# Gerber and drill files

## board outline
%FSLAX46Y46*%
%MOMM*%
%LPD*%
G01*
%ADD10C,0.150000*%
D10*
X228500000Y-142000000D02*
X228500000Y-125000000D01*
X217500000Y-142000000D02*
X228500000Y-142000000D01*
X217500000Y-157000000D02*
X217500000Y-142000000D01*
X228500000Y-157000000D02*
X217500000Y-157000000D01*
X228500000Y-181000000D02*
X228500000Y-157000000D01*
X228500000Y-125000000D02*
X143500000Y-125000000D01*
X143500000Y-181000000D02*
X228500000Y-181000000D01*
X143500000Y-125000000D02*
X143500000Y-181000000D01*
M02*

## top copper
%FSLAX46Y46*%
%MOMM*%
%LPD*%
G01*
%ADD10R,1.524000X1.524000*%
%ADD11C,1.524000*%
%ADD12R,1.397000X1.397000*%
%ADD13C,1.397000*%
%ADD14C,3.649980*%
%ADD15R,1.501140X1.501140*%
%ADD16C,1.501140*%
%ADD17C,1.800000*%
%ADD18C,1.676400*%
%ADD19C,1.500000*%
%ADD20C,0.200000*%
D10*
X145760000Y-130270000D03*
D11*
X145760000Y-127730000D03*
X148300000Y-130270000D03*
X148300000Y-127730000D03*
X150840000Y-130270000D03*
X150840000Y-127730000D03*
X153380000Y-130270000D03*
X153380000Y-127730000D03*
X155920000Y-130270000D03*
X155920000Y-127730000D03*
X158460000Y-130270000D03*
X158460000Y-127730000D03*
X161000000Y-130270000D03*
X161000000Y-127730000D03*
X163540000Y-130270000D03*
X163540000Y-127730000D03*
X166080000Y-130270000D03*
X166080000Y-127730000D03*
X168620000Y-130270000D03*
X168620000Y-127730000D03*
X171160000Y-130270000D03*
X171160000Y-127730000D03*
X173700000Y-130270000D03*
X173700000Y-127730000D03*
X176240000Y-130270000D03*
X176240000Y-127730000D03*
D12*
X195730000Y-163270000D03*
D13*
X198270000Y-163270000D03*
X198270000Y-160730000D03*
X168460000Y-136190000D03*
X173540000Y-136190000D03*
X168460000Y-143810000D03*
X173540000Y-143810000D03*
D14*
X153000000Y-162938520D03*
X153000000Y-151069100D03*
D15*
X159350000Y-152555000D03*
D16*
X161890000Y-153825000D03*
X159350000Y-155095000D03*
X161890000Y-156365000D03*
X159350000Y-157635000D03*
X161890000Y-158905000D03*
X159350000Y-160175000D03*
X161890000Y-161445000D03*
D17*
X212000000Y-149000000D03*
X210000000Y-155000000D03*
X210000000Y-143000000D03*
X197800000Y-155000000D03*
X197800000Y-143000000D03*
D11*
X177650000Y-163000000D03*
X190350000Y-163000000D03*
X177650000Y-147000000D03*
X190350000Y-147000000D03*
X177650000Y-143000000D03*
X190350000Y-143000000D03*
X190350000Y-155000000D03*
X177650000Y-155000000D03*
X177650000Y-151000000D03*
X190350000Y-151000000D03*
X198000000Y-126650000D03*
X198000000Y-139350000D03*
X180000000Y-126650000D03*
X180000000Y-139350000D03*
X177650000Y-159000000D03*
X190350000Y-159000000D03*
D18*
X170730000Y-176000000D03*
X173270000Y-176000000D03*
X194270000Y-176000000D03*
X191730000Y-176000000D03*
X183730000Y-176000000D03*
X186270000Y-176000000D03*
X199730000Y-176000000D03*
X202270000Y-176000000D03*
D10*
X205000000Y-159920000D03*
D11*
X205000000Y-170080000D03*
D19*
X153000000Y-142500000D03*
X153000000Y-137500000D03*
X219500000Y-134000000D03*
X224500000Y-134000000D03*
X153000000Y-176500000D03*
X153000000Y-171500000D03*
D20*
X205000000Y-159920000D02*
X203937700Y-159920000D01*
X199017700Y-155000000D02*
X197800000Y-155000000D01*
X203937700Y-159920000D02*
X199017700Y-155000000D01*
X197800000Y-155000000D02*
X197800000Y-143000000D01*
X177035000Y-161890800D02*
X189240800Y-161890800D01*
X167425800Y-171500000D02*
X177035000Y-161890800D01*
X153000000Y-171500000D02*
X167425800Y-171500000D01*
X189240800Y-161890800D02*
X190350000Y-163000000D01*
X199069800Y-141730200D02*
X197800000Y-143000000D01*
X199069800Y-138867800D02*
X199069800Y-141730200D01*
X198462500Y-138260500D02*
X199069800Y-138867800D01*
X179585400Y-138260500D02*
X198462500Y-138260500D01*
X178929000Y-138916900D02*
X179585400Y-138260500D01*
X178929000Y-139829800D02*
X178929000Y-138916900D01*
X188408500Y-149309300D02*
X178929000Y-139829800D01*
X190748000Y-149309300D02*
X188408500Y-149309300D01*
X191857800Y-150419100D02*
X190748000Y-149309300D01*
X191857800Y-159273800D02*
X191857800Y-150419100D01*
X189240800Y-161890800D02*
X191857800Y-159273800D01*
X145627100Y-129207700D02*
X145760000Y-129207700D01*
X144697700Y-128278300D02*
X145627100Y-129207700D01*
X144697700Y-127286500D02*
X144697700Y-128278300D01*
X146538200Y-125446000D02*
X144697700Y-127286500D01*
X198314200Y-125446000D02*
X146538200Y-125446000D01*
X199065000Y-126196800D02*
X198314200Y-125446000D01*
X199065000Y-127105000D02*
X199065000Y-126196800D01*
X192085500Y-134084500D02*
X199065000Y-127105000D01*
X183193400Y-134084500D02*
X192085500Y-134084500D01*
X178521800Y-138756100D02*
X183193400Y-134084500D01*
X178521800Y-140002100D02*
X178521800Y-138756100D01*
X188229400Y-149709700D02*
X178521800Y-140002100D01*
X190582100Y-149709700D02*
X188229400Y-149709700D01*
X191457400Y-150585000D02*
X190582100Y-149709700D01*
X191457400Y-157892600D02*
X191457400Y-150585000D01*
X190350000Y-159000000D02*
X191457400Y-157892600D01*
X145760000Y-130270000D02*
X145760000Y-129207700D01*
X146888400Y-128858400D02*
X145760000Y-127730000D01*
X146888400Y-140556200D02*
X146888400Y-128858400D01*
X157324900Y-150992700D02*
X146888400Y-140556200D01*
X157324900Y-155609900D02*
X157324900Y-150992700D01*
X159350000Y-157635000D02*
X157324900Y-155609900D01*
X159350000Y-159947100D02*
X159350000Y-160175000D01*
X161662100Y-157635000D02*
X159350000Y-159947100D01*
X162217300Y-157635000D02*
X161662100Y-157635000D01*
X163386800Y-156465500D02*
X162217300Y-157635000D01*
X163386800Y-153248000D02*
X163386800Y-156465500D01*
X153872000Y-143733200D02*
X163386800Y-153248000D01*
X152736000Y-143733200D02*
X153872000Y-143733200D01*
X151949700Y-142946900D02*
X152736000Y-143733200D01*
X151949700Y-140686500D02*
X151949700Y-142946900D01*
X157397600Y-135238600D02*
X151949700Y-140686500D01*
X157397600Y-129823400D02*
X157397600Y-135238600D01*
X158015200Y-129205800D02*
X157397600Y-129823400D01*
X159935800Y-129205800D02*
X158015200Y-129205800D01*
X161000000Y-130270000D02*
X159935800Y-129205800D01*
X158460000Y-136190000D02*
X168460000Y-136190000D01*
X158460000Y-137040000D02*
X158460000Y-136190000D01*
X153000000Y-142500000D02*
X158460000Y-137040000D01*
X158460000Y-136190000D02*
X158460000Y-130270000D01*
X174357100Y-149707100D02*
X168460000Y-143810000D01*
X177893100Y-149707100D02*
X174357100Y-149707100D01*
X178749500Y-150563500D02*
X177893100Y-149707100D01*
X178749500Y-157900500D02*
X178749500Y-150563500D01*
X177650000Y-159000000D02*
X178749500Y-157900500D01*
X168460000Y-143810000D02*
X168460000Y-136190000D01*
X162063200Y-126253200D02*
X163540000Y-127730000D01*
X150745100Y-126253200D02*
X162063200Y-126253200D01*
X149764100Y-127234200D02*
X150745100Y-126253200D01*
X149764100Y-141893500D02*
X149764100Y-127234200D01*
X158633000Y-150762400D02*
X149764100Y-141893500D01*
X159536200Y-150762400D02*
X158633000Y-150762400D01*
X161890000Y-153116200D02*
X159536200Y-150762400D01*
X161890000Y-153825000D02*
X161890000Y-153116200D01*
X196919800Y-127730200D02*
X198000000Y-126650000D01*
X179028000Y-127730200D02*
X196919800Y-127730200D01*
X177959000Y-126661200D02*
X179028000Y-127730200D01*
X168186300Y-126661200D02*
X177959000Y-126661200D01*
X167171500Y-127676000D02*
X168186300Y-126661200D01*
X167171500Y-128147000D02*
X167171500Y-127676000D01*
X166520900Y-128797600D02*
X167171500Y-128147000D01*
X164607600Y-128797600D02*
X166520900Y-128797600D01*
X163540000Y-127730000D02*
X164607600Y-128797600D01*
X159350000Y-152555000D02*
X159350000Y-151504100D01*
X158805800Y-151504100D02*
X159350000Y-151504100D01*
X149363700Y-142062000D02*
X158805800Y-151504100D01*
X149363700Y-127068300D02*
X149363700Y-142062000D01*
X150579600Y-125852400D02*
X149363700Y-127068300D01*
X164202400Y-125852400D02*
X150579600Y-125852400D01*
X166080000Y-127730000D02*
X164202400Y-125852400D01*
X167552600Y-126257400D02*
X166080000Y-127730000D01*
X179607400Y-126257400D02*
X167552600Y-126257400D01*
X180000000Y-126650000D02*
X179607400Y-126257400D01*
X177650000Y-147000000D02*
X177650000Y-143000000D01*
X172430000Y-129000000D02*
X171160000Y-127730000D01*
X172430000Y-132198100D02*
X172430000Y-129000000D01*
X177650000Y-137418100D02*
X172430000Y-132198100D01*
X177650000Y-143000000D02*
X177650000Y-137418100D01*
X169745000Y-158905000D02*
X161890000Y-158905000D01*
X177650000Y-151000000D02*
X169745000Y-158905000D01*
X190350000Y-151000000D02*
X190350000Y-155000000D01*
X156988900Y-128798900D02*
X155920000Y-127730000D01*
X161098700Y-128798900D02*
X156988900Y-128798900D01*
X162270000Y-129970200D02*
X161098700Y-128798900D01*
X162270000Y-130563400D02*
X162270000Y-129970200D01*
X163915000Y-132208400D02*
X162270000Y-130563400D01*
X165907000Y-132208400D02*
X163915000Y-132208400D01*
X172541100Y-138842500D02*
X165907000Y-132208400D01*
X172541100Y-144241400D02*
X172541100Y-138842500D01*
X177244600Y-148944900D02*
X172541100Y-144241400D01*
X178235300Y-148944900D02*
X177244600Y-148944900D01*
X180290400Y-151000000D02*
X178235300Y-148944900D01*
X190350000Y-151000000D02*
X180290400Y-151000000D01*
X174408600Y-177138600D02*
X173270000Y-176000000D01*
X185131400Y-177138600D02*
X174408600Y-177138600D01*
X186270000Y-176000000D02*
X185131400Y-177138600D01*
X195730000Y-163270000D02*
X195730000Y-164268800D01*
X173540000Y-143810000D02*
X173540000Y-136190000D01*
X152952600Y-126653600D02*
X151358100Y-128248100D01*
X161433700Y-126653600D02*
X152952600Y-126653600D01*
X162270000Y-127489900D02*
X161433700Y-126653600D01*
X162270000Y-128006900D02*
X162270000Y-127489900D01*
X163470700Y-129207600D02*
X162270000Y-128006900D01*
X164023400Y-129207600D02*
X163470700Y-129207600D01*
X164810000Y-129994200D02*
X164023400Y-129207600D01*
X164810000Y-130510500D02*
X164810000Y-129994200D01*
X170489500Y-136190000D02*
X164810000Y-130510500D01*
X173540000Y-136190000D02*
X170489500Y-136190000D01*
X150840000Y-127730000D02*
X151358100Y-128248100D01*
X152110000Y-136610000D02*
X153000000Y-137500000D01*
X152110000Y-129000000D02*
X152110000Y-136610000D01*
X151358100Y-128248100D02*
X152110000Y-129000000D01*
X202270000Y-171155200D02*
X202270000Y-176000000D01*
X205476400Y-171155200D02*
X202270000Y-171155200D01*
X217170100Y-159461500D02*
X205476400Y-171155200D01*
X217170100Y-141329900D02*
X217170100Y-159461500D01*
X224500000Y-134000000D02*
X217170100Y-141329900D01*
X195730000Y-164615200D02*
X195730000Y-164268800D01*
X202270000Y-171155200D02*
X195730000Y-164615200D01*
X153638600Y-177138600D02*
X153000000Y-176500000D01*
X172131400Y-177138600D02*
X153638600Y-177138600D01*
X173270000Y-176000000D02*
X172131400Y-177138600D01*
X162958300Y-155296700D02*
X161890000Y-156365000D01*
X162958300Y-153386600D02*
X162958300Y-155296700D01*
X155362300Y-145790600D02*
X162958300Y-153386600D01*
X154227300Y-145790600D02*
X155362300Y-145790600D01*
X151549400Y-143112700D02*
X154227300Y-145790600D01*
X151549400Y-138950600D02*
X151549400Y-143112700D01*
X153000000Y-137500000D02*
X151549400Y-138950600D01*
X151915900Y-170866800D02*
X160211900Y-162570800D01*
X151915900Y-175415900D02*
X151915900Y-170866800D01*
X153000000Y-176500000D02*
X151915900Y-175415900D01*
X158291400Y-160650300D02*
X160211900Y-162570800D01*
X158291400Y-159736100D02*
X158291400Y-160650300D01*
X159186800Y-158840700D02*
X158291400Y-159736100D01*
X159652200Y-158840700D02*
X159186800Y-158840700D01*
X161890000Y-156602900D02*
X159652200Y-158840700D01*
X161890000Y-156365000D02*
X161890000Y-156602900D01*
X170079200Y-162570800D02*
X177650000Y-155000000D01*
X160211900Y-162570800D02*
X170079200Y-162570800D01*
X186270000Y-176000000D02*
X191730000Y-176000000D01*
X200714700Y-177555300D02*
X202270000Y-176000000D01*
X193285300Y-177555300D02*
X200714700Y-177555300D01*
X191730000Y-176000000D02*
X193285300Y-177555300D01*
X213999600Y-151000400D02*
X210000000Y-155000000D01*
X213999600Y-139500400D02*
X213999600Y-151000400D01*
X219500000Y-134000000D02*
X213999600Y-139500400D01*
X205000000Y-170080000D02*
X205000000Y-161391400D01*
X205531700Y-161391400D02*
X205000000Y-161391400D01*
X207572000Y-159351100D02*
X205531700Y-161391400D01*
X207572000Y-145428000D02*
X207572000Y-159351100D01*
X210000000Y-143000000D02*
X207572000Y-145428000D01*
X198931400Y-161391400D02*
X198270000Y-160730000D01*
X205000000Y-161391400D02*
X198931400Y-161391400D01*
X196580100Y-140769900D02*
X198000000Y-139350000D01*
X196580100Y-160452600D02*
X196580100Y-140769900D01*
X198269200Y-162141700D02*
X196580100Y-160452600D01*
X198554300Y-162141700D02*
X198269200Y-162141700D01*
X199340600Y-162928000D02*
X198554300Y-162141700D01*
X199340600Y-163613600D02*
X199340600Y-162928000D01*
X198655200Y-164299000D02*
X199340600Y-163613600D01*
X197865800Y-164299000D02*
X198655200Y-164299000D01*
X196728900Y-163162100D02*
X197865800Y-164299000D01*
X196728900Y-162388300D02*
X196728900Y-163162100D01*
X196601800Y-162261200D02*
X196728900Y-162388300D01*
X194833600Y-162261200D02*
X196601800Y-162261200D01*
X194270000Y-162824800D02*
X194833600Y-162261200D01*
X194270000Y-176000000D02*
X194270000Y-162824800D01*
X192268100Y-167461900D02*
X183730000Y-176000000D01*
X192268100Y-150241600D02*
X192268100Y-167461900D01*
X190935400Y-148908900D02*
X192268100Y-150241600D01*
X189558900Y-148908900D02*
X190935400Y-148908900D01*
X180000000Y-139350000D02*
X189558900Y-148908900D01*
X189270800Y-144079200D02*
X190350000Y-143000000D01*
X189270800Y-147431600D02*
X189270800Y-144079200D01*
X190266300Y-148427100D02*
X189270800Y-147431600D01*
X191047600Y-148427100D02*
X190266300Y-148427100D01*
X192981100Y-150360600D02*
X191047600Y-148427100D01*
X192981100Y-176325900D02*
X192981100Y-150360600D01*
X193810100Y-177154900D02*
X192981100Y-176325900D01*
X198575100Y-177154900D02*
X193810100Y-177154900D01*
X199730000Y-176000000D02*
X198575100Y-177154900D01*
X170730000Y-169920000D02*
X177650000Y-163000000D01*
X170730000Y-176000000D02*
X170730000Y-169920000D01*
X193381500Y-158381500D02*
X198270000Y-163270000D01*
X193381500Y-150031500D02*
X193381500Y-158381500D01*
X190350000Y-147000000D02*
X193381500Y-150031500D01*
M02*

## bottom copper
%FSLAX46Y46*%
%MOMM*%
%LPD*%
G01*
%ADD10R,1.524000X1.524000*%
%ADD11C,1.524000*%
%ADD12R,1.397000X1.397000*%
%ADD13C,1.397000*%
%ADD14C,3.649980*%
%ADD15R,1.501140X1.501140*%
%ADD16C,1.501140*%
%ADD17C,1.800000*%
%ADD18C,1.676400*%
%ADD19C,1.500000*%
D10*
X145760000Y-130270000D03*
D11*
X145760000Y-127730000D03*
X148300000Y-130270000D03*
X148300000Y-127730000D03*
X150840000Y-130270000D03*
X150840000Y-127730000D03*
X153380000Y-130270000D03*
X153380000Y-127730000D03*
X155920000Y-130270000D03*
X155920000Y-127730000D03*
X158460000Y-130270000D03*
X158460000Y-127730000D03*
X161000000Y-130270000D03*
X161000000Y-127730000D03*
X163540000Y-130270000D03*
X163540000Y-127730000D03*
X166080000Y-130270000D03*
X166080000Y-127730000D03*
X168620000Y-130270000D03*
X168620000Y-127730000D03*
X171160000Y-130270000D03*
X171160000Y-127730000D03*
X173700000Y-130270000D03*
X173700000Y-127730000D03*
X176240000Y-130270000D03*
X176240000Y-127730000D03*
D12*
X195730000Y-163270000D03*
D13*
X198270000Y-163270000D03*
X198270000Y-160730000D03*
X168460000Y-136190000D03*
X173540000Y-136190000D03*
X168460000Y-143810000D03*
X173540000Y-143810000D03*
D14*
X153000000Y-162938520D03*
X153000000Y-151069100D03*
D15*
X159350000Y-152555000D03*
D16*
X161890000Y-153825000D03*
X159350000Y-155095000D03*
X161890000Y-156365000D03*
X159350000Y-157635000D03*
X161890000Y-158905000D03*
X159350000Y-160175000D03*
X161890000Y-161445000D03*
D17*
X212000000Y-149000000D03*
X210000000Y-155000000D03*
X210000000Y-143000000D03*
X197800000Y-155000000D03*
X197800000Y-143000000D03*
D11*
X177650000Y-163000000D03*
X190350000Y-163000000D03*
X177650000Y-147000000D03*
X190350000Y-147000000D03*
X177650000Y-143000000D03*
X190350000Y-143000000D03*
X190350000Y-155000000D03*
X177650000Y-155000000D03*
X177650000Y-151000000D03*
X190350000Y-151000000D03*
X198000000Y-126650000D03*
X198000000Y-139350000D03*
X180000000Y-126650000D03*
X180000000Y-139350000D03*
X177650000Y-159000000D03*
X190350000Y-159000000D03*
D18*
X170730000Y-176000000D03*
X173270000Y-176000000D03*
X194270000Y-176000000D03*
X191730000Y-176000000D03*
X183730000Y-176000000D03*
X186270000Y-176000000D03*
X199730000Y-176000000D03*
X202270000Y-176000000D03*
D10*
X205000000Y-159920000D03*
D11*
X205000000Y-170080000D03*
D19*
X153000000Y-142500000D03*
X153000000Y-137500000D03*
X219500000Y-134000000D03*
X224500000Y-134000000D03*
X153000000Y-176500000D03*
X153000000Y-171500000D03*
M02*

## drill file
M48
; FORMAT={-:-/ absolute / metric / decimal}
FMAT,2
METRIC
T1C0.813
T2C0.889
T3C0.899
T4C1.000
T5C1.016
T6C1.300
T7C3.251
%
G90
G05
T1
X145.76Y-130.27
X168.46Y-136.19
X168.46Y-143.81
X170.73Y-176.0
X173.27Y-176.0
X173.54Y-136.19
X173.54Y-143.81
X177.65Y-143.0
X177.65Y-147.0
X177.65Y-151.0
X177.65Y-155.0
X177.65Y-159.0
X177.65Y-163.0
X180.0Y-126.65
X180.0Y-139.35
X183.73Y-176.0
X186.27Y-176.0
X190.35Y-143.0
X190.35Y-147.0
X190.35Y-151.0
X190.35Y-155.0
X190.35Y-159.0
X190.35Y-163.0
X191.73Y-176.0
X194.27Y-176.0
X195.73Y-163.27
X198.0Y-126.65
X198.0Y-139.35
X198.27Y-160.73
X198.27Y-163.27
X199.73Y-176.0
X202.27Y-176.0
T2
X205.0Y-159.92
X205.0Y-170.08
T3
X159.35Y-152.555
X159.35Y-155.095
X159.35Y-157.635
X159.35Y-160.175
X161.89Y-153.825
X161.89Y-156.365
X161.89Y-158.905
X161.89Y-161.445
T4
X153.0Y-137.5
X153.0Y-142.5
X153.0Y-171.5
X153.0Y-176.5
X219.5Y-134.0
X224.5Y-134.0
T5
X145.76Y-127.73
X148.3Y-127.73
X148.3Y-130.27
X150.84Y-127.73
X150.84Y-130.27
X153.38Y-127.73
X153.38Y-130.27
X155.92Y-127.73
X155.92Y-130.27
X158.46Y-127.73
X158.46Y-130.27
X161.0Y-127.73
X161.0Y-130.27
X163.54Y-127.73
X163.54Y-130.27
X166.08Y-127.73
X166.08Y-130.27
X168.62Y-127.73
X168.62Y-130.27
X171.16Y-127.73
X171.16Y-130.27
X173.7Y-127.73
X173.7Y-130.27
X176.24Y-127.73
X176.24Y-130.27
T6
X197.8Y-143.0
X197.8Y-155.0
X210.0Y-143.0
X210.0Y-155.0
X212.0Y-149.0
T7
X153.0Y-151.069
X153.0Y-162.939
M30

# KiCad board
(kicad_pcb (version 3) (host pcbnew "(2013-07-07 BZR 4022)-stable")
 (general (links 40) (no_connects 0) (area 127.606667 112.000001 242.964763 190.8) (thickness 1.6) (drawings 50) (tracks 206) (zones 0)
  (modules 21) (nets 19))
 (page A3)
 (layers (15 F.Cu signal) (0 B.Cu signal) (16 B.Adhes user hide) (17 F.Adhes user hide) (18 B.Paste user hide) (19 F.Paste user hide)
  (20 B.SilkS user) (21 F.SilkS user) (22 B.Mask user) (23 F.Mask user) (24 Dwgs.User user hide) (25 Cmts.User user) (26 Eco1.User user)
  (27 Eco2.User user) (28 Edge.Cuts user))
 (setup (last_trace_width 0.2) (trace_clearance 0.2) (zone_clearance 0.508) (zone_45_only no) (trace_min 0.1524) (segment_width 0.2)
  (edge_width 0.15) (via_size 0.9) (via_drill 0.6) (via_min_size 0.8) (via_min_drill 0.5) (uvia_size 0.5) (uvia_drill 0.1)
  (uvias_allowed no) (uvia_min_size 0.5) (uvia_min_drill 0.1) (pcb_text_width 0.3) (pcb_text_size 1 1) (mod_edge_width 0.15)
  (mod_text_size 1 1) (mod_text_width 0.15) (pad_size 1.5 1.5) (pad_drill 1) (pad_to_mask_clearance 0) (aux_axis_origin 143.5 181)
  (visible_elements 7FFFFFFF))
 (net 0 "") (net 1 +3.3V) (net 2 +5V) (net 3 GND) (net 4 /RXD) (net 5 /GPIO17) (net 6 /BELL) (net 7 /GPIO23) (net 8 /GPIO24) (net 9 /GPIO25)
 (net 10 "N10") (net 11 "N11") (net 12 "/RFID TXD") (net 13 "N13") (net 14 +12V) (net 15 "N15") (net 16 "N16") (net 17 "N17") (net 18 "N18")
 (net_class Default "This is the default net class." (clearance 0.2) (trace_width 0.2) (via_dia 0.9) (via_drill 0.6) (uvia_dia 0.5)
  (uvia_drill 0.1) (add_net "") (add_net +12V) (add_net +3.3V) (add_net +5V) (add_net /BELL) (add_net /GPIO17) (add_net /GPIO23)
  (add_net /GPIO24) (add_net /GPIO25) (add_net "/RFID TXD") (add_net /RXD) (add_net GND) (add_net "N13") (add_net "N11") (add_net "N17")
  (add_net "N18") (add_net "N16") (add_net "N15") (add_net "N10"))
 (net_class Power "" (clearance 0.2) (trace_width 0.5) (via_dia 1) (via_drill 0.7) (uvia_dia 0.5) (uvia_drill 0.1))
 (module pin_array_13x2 (layer F.Cu) (at 161 129)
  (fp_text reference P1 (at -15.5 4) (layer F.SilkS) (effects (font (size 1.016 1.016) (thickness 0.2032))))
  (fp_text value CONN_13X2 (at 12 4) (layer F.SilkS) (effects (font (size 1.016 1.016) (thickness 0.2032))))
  (pad 1 thru_hole rect (at -15.24 1.27) (size 1.524 1.524) (drill 0.8128) (layers *.Cu *.Mask F.SilkS) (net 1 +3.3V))
  (pad 2 thru_hole circle (at -15.24 -1.27) (size 1.524 1.524) (drill 1.016) (layers *.Cu *.Mask F.SilkS) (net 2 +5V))
  (pad 3 thru_hole circle (at -12.7 1.27) (size 1.524 1.524) (drill 1.016) (layers *.Cu *.Mask F.SilkS))
  (pad 4 thru_hole circle (at -12.7 -1.27) (size 1.524 1.524) (drill 1.016) (layers *.Cu *.Mask F.SilkS))
  (pad 5 thru_hole circle (at -10.16 1.27) (size 1.524 1.524) (drill 1.016) (layers *.Cu *.Mask F.SilkS))
  (pad 6 thru_hole circle (at -10.16 -1.27) (size 1.524 1.524) (drill 1.016) (layers *.Cu *.Mask F.SilkS) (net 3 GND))
  (pad 7 thru_hole circle (at -7.62 1.27) (size 1.524 1.524) (drill 1.016) (layers *.Cu *.Mask F.SilkS))
  (pad 8 thru_hole circle (at -7.62 -1.27) (size 1.524 1.524) (drill 1.016) (layers *.Cu *.Mask F.SilkS))
  (pad 9 thru_hole circle (at -5.08 1.27) (size 1.524 1.524) (drill 1.016) (layers *.Cu *.Mask F.SilkS))
  (pad 10 thru_hole circle (at -5.08 -1.27) (size 1.524 1.524) (drill 1.016) (layers *.Cu *.Mask F.SilkS) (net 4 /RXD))
  (pad 11 thru_hole circle (at -2.54 1.27) (size 1.524 1.524) (drill 1.016) (layers *.Cu *.Mask F.SilkS) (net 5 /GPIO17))
  (pad 12 thru_hole circle (at -2.54 -1.27) (size 1.524 1.524) (drill 1.016) (layers *.Cu *.Mask F.SilkS))
  (pad 13 thru_hole circle (at 0 1.27) (size 1.524 1.524) (drill 1.016) (layers *.Cu *.Mask F.SilkS) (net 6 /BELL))
  (pad 14 thru_hole circle (at 0 -1.27) (size 1.524 1.524) (drill 1.016) (layers *.Cu *.Mask F.SilkS))
  (pad 15 thru_hole circle (at 2.54 1.27) (size 1.524 1.524) (drill 1.016) (layers *.Cu *.Mask F.SilkS))
  (pad 16 thru_hole circle (at 2.54 -1.27) (size 1.524 1.524) (drill 1.016) (layers *.Cu *.Mask F.SilkS) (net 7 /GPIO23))
  (pad 17 thru_hole circle (at 5.08 1.27) (size 1.524 1.524) (drill 1.016) (layers *.Cu *.Mask F.SilkS))
  (pad 18 thru_hole circle (at 5.08 -1.27) (size 1.524 1.524) (drill 1.016) (layers *.Cu *.Mask F.SilkS) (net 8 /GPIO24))
  (pad 19 thru_hole circle (at 7.62 1.27) (size 1.524 1.524) (drill 1.016) (layers *.Cu *.Mask F.SilkS))
  (pad 20 thru_hole circle (at 7.62 -1.27) (size 1.524 1.524) (drill 1.016) (layers *.Cu *.Mask F.SilkS))
  (pad 21 thru_hole circle (at 10.16 1.27) (size 1.524 1.524) (drill 1.016) (layers *.Cu *.Mask F.SilkS))
  (pad 22 thru_hole circle (at 10.16 -1.27) (size 1.524 1.524) (drill 1.016) (layers *.Cu *.Mask F.SilkS) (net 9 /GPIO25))
  (pad 23 thru_hole circle (at 12.7 1.27) (size 1.524 1.524) (drill 1.016) (layers *.Cu *.Mask F.SilkS))
  (pad 24 thru_hole circle (at 12.7 -1.27) (size 1.524 1.524) (drill 1.016) (layers *.Cu *.Mask F.SilkS))
  (pad 25 thru_hole circle (at 15.24 1.27) (size 1.524 1.524) (drill 1.016) (layers *.Cu *.Mask F.SilkS))
  (pad 26 thru_hole circle (at 15.24 -1.27) (size 1.524 1.524) (drill 1.016) (layers *.Cu *.Mask F.SilkS)))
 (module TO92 (layer F.Cu) (at 197 162 180)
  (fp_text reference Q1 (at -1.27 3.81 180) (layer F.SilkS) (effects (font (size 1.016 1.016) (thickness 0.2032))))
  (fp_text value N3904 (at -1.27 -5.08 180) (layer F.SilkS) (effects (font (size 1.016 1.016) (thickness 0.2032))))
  (pad 1 thru_hole rect (at 1.27 -1.27 180) (size 1.397 1.397) (drill 0.8128) (layers *.Cu *.Mask F.SilkS) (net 3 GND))
  (pad 2 thru_hole circle (at -1.27 -1.27 180) (size 1.397 1.397) (drill 0.8128) (layers *.Cu *.Mask F.SilkS) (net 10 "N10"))
  (pad 3 thru_hole circle (at -1.27 1.27 180) (size 1.397 1.397) (drill 0.8128) (layers *.Cu *.Mask F.SilkS) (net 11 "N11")))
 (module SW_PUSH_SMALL (layer F.Cu) (at 171 140 90)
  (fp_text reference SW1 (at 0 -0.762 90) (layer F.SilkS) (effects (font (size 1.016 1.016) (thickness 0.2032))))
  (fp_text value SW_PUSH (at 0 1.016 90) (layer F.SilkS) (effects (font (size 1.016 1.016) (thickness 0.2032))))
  (pad 1 thru_hole circle (at 3.81 -2.54 90) (size 1.397 1.397) (drill 0.8128) (layers *.Cu *.Mask F.SilkS) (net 5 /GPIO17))
  (pad 2 thru_hole circle (at 3.81 2.54 90) (size 1.397 1.397) (drill 0.8128) (layers *.Cu *.Mask F.SilkS) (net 3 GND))
  (pad 1 thru_hole circle (at -3.81 -2.54 90) (size 1.397 1.397) (drill 0.8128) (layers *.Cu *.Mask F.SilkS) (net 5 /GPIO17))
  (pad 2 thru_hole circle (at -3.81 2.54 90) (size 1.397 1.397) (drill 0.8128) (layers *.Cu *.Mask F.SilkS) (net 3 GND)))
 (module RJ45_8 (layer F.Cu) (at 153 157 270)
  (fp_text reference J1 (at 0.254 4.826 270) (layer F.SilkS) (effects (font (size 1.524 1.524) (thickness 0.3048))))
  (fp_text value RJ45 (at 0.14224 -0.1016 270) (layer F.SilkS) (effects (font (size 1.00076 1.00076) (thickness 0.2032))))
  (pad Hole np_thru_hole circle (at 5.93852 0 270) (size 3.64998 3.64998) (drill 3.2512) (layers *.Cu *.SilkS *.Mask))
  (pad Hole np_thru_hole circle (at -5.9309 0 270) (size 3.64998 3.64998) (drill 3.2512) (layers *.Cu *.SilkS *.Mask))
  (pad 1 thru_hole rect (at -4.445 -6.35 270) (size 1.50114 1.50114) (drill 0.89916) (layers *.Cu *.Mask F.SilkS) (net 8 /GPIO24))
  (pad 2 thru_hole circle (at -3.175 -8.89 270) (size 1.50114 1.50114) (drill 0.89916) (layers *.Cu *.Mask F.SilkS) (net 7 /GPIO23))
  (pad 3 thru_hole circle (at -1.905 -6.35 270) (size 1.50114 1.50114) (drill 0.89916) (layers *.Cu *.Mask F.SilkS))
  (pad 4 thru_hole circle (at -0.635 -8.89 270) (size 1.50114 1.50114) (drill 0.89916) (layers *.Cu *.Mask F.SilkS) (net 3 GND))
  (pad 5 thru_hole circle (at 0.635 -6.35 270) (size 1.50114 1.50114) (drill 0.89916) (layers *.Cu *.Mask F.SilkS) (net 2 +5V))
  (pad 6 thru_hole circle (at 1.905 -8.89 270) (size 1.50114 1.50114) (drill 0.89916) (layers *.Cu *.Mask F.SilkS) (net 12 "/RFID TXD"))
  (pad 7 thru_hole circle (at 3.175 -6.35 270) (size 1.50114 1.50114) (drill 0.89916) (layers *.Cu *.Mask F.SilkS) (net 6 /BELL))
  (pad 8 thru_hole circle (at 4.445 -8.89 270) (size 1.50114 1.50114) (drill 0.89916) (layers *.Cu *.Mask F.SilkS)))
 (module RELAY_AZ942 (layer F.Cu) (at 210 149 180)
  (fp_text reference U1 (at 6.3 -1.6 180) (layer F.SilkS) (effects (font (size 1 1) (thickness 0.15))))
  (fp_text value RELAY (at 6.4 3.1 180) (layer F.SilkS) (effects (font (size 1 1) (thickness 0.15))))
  (pad 1 thru_hole circle (at -2 0 180) (size 1.8 1.8) (drill 1.3) (layers *.Cu *.Mask F.SilkS))
  (pad 2 thru_hole circle (at 0 -6 180) (size 1.8 1.8) (drill 1.3) (layers *.Cu *.Mask F.SilkS) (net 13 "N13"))
  (pad 5 thru_hole circle (at 0 6 180) (size 1.8 1.8) (drill 1.3) (layers *.Cu *.Mask F.SilkS) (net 11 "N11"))
  (pad 3 thru_hole circle (at 12.2 -6 180) (size 1.8 1.8) (drill 1.3) (layers *.Cu *.Mask F.SilkS) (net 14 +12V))
  (pad 4 thru_hole circle (at 12.2 6 180) (size 1.8 1.8) (drill 1.3) (layers *.Cu *.Mask F.SilkS) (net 14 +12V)))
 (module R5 (layer F.Cu) (at 184 163) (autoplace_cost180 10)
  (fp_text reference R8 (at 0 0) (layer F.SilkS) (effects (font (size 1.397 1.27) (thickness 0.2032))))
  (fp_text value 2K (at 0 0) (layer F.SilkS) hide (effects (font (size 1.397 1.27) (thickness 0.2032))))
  (pad 1 thru_hole circle (at -6.35 0) (size 1.524 1.524) (drill 0.8128) (layers *.Cu *.Mask F.SilkS) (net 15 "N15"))
  (pad 2 thru_hole circle (at 6.35 0) (size 1.524 1.524) (drill 0.8128) (layers *.Cu *.Mask F.SilkS) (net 14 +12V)))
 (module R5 (layer F.Cu) (at 184 147) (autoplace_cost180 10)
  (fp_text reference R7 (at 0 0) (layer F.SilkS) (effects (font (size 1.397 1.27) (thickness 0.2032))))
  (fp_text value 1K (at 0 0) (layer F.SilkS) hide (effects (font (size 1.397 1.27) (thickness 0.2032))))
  (pad 1 thru_hole circle (at -6.35 0) (size 1.524 1.524) (drill 0.8128) (layers *.Cu *.Mask F.SilkS) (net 9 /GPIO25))
  (pad 2 thru_hole circle (at 6.35 0) (size 1.524 1.524) (drill 0.8128) (layers *.Cu *.Mask F.SilkS) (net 10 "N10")))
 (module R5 (layer F.Cu) (at 184 143) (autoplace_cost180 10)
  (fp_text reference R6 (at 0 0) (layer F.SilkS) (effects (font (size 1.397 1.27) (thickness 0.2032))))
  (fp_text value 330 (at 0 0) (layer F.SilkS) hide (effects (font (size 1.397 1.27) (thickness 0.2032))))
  (pad 1 thru_hole circle (at -6.35 0) (size 1.524 1.524) (drill 0.8128) (layers *.Cu *.Mask F.SilkS) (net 9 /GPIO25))
  (pad 2 thru_hole circle (at 6.35 0) (size 1.524 1.524) (drill 0.8128) (layers *.Cu *.Mask F.SilkS) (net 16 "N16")))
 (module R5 (layer F.Cu) (at 184 155 180) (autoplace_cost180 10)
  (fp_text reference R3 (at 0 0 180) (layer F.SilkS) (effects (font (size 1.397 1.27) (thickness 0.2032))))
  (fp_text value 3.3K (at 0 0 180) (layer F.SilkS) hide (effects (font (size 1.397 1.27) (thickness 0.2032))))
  (pad 1 thru_hole circle (at -6.35 0 180) (size 1.524 1.524) (drill 0.8128) (layers *.Cu *.Mask F.SilkS) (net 4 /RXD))
  (pad 2 thru_hole circle (at 6.35 0 180) (size 1.524 1.524) (drill 0.8128) (layers *.Cu *.Mask F.SilkS) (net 3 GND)))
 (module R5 (layer F.Cu) (at 184 151) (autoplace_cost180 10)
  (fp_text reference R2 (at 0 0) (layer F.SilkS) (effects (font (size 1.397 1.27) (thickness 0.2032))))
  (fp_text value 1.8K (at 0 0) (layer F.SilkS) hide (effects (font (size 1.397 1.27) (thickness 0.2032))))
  (pad 1 thru_hole circle (at -6.35 0) (size 1.524 1.524) (drill 0.8128) (layers *.Cu *.Mask F.SilkS) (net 12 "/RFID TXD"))
  (pad 2 thru_hole circle (at 6.35 0) (size 1.524 1.524) (drill 0.8128) (layers *.Cu *.Mask F.SilkS) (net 4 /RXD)))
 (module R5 (layer F.Cu) (at 198 133 270) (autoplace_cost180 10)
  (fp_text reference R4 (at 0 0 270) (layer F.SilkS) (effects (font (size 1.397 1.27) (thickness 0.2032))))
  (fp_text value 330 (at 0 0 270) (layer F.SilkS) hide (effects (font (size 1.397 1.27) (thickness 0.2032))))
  (pad 1 thru_hole circle (at -6.35 0 270) (size 1.524 1.524) (drill 0.8128) (layers *.Cu *.Mask F.SilkS) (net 7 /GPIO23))
  (pad 2 thru_hole circle (at 6.35 0 270) (size 1.524 1.524) (drill 0.8128) (layers *.Cu *.Mask F.SilkS) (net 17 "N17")))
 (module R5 (layer F.Cu) (at 180 133 270) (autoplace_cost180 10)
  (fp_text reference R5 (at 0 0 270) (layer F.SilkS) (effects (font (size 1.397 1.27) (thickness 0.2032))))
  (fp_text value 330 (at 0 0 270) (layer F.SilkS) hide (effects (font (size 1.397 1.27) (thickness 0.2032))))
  (pad 1 thru_hole circle (at -6.35 0 270) (size 1.524 1.524) (drill 0.8128) (layers *.Cu *.Mask F.SilkS) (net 8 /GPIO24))
  (pad 2 thru_hole circle (at 6.35 0 270) (size 1.524 1.524) (drill 0.8128) (layers *.Cu *.Mask F.SilkS) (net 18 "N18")))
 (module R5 (layer F.Cu) (at 184 159) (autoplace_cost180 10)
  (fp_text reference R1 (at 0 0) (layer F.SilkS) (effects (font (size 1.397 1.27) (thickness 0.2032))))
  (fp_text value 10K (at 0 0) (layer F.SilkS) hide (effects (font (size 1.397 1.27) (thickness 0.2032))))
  (pad 1 thru_hole circle (at -6.35 0) (size 1.524 1.524) (drill 0.8128) (layers *.Cu *.Mask F.SilkS) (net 5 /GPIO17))
  (pad 2 thru_hole circle (at 6.35 0) (size 1.524 1.524) (drill 0.8128) (layers *.Cu *.Mask F.SilkS) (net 1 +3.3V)))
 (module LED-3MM (layer F.Cu) (at 172 176)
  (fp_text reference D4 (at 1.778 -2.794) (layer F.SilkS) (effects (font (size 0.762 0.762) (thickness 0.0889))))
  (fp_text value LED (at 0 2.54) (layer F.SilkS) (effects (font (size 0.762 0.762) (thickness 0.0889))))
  (pad 1 thru_hole circle (at -1.27 0) (size 1.6764 1.6764) (drill 0.8128) (layers *.Cu *.Mask F.SilkS) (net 15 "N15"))
  (pad 2 thru_hole circle (at 1.27 0) (size 1.6764 1.6764) (drill 0.8128) (layers *.Cu *.Mask F.SilkS) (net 3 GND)))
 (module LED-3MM (layer F.Cu) (at 193 176 180)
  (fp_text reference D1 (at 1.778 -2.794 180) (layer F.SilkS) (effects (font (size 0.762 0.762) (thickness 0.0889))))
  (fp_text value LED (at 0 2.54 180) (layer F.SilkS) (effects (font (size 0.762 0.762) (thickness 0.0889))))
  (pad 1 thru_hole circle (at -1.27 0 180) (size 1.6764 1.6764) (drill 0.8128) (layers *.Cu *.Mask F.SilkS) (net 17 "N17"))
  (pad 2 thru_hole circle (at 1.27 0 180) (size 1.6764 1.6764) (drill 0.8128) (layers *.Cu *.Mask F.SilkS) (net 3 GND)))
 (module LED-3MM (layer F.Cu) (at 185 176)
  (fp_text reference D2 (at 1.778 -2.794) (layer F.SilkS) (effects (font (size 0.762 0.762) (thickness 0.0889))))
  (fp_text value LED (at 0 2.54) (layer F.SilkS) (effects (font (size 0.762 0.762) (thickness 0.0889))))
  (pad 1 thru_hole circle (at -1.27 0) (size 1.6764 1.6764) (drill 0.8128) (layers *.Cu *.Mask F.SilkS) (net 18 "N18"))
  (pad 2 thru_hole circle (at 1.27 0) (size 1.6764 1.6764) (drill 0.8128) (layers *.Cu *.Mask F.SilkS) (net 3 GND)))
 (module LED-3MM (layer F.Cu) (at 201 176)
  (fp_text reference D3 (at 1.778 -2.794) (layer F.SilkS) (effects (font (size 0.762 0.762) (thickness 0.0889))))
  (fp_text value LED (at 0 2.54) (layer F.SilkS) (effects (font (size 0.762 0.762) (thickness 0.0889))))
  (pad 1 thru_hole circle (at -1.27 0) (size 1.6764 1.6764) (drill 0.8128) (layers *.Cu *.Mask F.SilkS) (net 16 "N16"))
  (pad 2 thru_hole circle (at 1.27 0) (size 1.6764 1.6764) (drill 0.8128) (layers *.Cu *.Mask F.SilkS) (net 3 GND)))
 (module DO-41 (layer F.Cu) (at 205 165 90)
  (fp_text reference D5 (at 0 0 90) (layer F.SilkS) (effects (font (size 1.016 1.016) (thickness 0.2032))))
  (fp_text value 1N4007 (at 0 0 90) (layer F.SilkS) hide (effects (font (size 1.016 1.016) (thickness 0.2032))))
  (pad 2 thru_hole rect (at 5.08 0 90) (size 1.524 1.524) (drill 0.889) (layers *.Cu *.Mask F.SilkS) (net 14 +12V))
  (pad 1 thru_hole circle (at -5.08 0 90) (size 1.524 1.524) (drill 0.889) (layers *.Cu *.Mask F.SilkS) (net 11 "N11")))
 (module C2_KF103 (layer F.Cu) (at 153 140 90)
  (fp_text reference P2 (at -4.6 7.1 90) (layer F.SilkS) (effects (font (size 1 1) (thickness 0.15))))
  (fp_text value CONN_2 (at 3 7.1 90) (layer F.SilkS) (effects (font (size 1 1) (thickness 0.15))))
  (pad 1 thru_hole circle (at -2.5 0 90) (size 1.5 1.5) (drill 1) (layers *.Cu *.Mask F.SilkS) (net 5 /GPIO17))
  (pad 2 thru_hole circle (at 2.5 0 90) (size 1.5 1.5) (drill 1) (layers *.Cu *.Mask F.SilkS) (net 3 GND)))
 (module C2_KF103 (layer F.Cu) (at 222 134)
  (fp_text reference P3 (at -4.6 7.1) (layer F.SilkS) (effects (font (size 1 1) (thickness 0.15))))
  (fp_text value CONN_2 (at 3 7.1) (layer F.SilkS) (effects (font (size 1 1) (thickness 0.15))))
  (pad 1 thru_hole circle (at -2.5 0) (size 1.5 1.5) (drill 1) (layers *.Cu *.Mask F.SilkS) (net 13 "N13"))
  (pad 2 thru_hole circle (at 2.5 0) (size 1.5 1.5) (drill 1) (layers *.Cu *.Mask F.SilkS) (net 3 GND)))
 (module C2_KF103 (layer F.Cu) (at 153 174 90)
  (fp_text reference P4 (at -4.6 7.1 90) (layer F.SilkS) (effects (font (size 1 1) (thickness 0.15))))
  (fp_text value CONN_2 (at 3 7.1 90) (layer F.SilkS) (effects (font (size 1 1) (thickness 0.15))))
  (pad 1 thru_hole circle (at -2.5 0 90) (size 1.5 1.5) (drill 1) (layers *.Cu *.Mask F.SilkS) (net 3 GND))
  (pad 2 thru_hole circle (at 2.5 0 90) (size 1.5 1.5) (drill 1) (layers *.Cu *.Mask F.SilkS) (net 14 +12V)))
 (gr_line (start 228.5 142) (end 228.5 125) (angle 90) (layer Edge.Cuts) (width 0.15))
 (gr_line (start 217.5 142) (end 228.5 142) (angle 90) (layer Edge.Cuts) (width 0.15))
 (gr_line (start 217.5 157) (end 217.5 142) (angle 90) (layer Edge.Cuts) (width 0.15))
 (gr_line (start 228.5 157) (end 217.5 157) (angle 90) (layer Edge.Cuts) (width 0.15))
 (gr_line (start 228.5 181) (end 228.5 157) (angle 90) (layer Edge.Cuts) (width 0.15))
 (gr_line (start 228.5 125) (end 143.5 125) (angle 90) (layer Edge.Cuts) (width 0.15))
 (gr_line (start 143.5 181) (end 228.5 181) (angle 90) (layer Edge.Cuts) (width 0.15))
 (gr_line (start 143.5 125) (end 143.5 181) (angle 90) (layer Edge.Cuts) (width 0.15))
 (segment (start 205 159.92) (end 203.9377 159.92) (width 0.2) (layer F.Cu) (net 14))
 (segment (start 199.0177 155) (end 197.8 155) (width 0.2) (layer F.Cu) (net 14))
 (segment (start 203.9377 159.92) (end 199.0177 155) (width 0.2) (layer F.Cu) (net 14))
 (segment (start 197.8 155) (end 197.8 143) (width 0.2) (layer F.Cu) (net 14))
 (segment (start 177.035 161.8908) (end 189.2408 161.8908) (width 0.2) (layer F.Cu) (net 14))
 (segment (start 167.4258 171.5) (end 177.035 161.8908) (width 0.2) (layer F.Cu) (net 14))
 (segment (start 153 171.5) (end 167.4258 171.5) (width 0.2) (layer F.Cu) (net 14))
 (segment (start 189.2408 161.8908) (end 190.35 163) (width 0.2) (layer F.Cu) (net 14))
 (segment (start 199.0698 141.7302) (end 197.8 143) (width 0.2) (layer F.Cu) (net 14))
 (segment (start 199.0698 138.8678) (end 199.0698 141.7302) (width 0.2) (layer F.Cu) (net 14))
 (segment (start 198.4625 138.2605) (end 199.0698 138.8678) (width 0.2) (layer F.Cu) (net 14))
 (segment (start 179.5854 138.2605) (end 198.4625 138.2605) (width 0.2) (layer F.Cu) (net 14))
 (segment (start 178.929 138.9169) (end 179.5854 138.2605) (width 0.2) (layer F.Cu) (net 14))
 (segment (start 178.929 139.8298) (end 178.929 138.9169) (width 0.2) (layer F.Cu) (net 14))
 (segment (start 188.4085 149.3093) (end 178.929 139.8298) (width 0.2) (layer F.Cu) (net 14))
 (segment (start 190.748 149.3093) (end 188.4085 149.3093) (width 0.2) (layer F.Cu) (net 14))
 (segment (start 191.8578 150.4191) (end 190.748 149.3093) (width 0.2) (layer F.Cu) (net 14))
 (segment (start 191.8578 159.2738) (end 191.8578 150.4191) (width 0.2) (layer F.Cu) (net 14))
 (segment (start 189.2408 161.8908) (end 191.8578 159.2738) (width 0.2) (layer F.Cu) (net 14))
 (segment (start 145.6271 129.2077) (end 145.76 129.2077) (width 0.2) (layer F.Cu) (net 1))
 (segment (start 144.6977 128.2783) (end 145.6271 129.2077) (width 0.2) (layer F.Cu) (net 1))
 (segment (start 144.6977 127.2865) (end 144.6977 128.2783) (width 0.2) (layer F.Cu) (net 1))
 (segment (start 146.5382 125.446) (end 144.6977 127.2865) (width 0.2) (layer F.Cu) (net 1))
 (segment (start 198.3142 125.446) (end 146.5382 125.446) (width 0.2) (layer F.Cu) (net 1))
 (segment (start 199.065 126.1968) (end 198.3142 125.446) (width 0.2) (layer F.Cu) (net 1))
 (segment (start 199.065 127.105) (end 199.065 126.1968) (width 0.2) (layer F.Cu) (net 1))
 (segment (start 192.0855 134.0845) (end 199.065 127.105) (width 0.2) (layer F.Cu) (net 1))
 (segment (start 183.1934 134.0845) (end 192.0855 134.0845) (width 0.2) (layer F.Cu) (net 1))
 (segment (start 178.5218 138.7561) (end 183.1934 134.0845) (width 0.2) (layer F.Cu) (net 1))
 (segment (start 178.5218 140.0021) (end 178.5218 138.7561) (width 0.2) (layer F.Cu) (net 1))
 (segment (start 188.2294 149.7097) (end 178.5218 140.0021) (width 0.2) (layer F.Cu) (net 1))
 (segment (start 190.5821 149.7097) (end 188.2294 149.7097) (width 0.2) (layer F.Cu) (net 1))
 (segment (start 191.4574 150.585) (end 190.5821 149.7097) (width 0.2) (layer F.Cu) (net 1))
 (segment (start 191.4574 157.8926) (end 191.4574 150.585) (width 0.2) (layer F.Cu) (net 1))
 (segment (start 190.35 159) (end 191.4574 157.8926) (width 0.2) (layer F.Cu) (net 1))
 (segment (start 145.76 130.27) (end 145.76 129.2077) (width 0.2) (layer F.Cu) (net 1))
 (segment (start 146.8884 128.8584) (end 145.76 127.73) (width 0.2) (layer F.Cu) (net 2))
 (segment (start 146.8884 140.5562) (end 146.8884 128.8584) (width 0.2) (layer F.Cu) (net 2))
 (segment (start 157.3249 150.9927) (end 146.8884 140.5562) (width 0.2) (layer F.Cu) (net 2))
 (segment (start 157.3249 155.6099) (end 157.3249 150.9927) (width 0.2) (layer F.Cu) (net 2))
 (segment (start 159.35 157.635) (end 157.3249 155.6099) (width 0.2) (layer F.Cu) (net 2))
 (segment (start 159.35 159.9471) (end 159.35 160.175) (width 0.2) (layer F.Cu) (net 6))
 (segment (start 161.6621 157.635) (end 159.35 159.9471) (width 0.2) (layer F.Cu) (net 6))
 (segment (start 162.2173 157.635) (end 161.6621 157.635) (width 0.2) (layer F.Cu) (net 6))
 (segment (start 163.3868 156.4655) (end 162.2173 157.635) (width 0.2) (layer F.Cu) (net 6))
 (segment (start 163.3868 153.248) (end 163.3868 156.4655) (width 0.2) (layer F.Cu) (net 6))
 (segment (start 153.872 143.7332) (end 163.3868 153.248) (width 0.2) (layer F.Cu) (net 6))
 (segment (start 152.736 143.7332) (end 153.872 143.7332) (width 0.2) (layer F.Cu) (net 6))
 (segment (start 151.9497 142.9469) (end 152.736 143.7332) (width 0.2) (layer F.Cu) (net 6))
 (segment (start 151.9497 140.6865) (end 151.9497 142.9469) (width 0.2) (layer F.Cu) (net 6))
 (segment (start 157.3976 135.2386) (end 151.9497 140.6865) (width 0.2) (layer F.Cu) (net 6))
 (segment (start 157.3976 129.8234) (end 157.3976 135.2386) (width 0.2) (layer F.Cu) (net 6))
 (segment (start 158.0152 129.2058) (end 157.3976 129.8234) (width 0.2) (layer F.Cu) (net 6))
 (segment (start 159.9358 129.2058) (end 158.0152 129.2058) (width 0.2) (layer F.Cu) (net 6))
 (segment (start 161 130.27) (end 159.9358 129.2058) (width 0.2) (layer F.Cu) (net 6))
 (segment (start 158.46 136.19) (end 168.46 136.19) (width 0.2) (layer F.Cu) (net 5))
 (segment (start 158.46 137.04) (end 158.46 136.19) (width 0.2) (layer F.Cu) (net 5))
 (segment (start 153 142.5) (end 158.46 137.04) (width 0.2) (layer F.Cu) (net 5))
 (segment (start 158.46 136.19) (end 158.46 130.27) (width 0.2) (layer F.Cu) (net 5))
 (segment (start 174.3571 149.7071) (end 168.46 143.81) (width 0.2) (layer F.Cu) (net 5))
 (segment (start 177.8931 149.7071) (end 174.3571 149.7071) (width 0.2) (layer F.Cu) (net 5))
 (segment (start 178.7495 150.5635) (end 177.8931 149.7071) (width 0.2) (layer F.Cu) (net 5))
 (segment (start 178.7495 157.9005) (end 178.7495 150.5635) (width 0.2) (layer F.Cu) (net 5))
 (segment (start 177.65 159) (end 178.7495 157.9005) (width 0.2) (layer F.Cu) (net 5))
 (segment (start 168.46 143.81) (end 168.46 136.19) (width 0.2) (layer F.Cu) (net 5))
 (segment (start 162.0632 126.2532) (end 163.54 127.73) (width 0.2) (layer F.Cu) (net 7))
 (segment (start 150.7451 126.2532) (end 162.0632 126.2532) (width 0.2) (layer F.Cu) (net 7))
 (segment (start 149.7641 127.2342) (end 150.7451 126.2532) (width 0.2) (layer F.Cu) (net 7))
 (segment (start 149.7641 141.8935) (end 149.7641 127.2342) (width 0.2) (layer F.Cu) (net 7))
 (segment (start 158.633 150.7624) (end 149.7641 141.8935) (width 0.2) (layer F.Cu) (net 7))
 (segment (start 159.5362 150.7624) (end 158.633 150.7624) (width 0.2) (layer F.Cu) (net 7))
 (segment (start 161.89 153.1162) (end 159.5362 150.7624) (width 0.2) (layer F.Cu) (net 7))
 (segment (start 161.89 153.825) (end 161.89 153.1162) (width 0.2) (layer F.Cu) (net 7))
 (segment (start 196.9198 127.7302) (end 198 126.65) (width 0.2) (layer F.Cu) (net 7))
 (segment (start 179.028 127.7302) (end 196.9198 127.7302) (width 0.2) (layer F.Cu) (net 7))
 (segment (start 177.959 126.6612) (end 179.028 127.7302) (width 0.2) (layer F.Cu) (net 7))
 (segment (start 168.1863 126.6612) (end 177.959 126.6612) (width 0.2) (layer F.Cu) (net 7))
 (segment (start 167.1715 127.676) (end 168.1863 126.6612) (width 0.2) (layer F.Cu) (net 7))
 (segment (start 167.1715 128.147) (end 167.1715 127.676) (width 0.2) (layer F.Cu) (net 7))
 (segment (start 166.5209 128.7976) (end 167.1715 128.147) (width 0.2) (layer F.Cu) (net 7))
 (segment (start 164.6076 128.7976) (end 166.5209 128.7976) (width 0.2) (layer F.Cu) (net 7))
 (segment (start 163.54 127.73) (end 164.6076 128.7976) (width 0.2) (layer F.Cu) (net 7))
 (segment (start 159.35 152.555) (end 159.35 151.5041) (width 0.2) (layer F.Cu) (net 8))
 (segment (start 158.8058 151.5041) (end 159.35 151.5041) (width 0.2) (layer F.Cu) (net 8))
 (segment (start 149.3637 142.062) (end 158.8058 151.5041) (width 0.2) (layer F.Cu) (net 8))
 (segment (start 149.3637 127.0683) (end 149.3637 142.062) (width 0.2) (layer F.Cu) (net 8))
 (segment (start 150.5796 125.8524) (end 149.3637 127.0683) (width 0.2) (layer F.Cu) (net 8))
 (segment (start 164.2024 125.8524) (end 150.5796 125.8524) (width 0.2) (layer F.Cu) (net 8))
 (segment (start 166.08 127.73) (end 164.2024 125.8524) (width 0.2) (layer F.Cu) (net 8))
 (segment (start 167.5526 126.2574) (end 166.08 127.73) (width 0.2) (layer F.Cu) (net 8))
 (segment (start 179.6074 126.2574) (end 167.5526 126.2574) (width 0.2) (layer F.Cu) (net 8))
 (segment (start 180 126.65) (end 179.6074 126.2574) (width 0.2) (layer F.Cu) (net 8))
 (segment (start 177.65 147) (end 177.65 143) (width 0.2) (layer F.Cu) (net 9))
 (segment (start 172.43 129) (end 171.16 127.73) (width 0.2) (layer F.Cu) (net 9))
 (segment (start 172.43 132.1981) (end 172.43 129) (width 0.2) (layer F.Cu) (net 9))
 (segment (start 177.65 137.4181) (end 172.43 132.1981) (width 0.2) (layer F.Cu) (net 9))
 (segment (start 177.65 143) (end 177.65 137.4181) (width 0.2) (layer F.Cu) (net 9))
 (segment (start 169.745 158.905) (end 161.89 158.905) (width 0.2) (layer F.Cu) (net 12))
 (segment (start 177.65 151) (end 169.745 158.905) (width 0.2) (layer F.Cu) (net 12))
 (segment (start 190.35 151) (end 190.35 155) (width 0.2) (layer F.Cu) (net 4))
 (segment (start 156.9889 128.7989) (end 155.92 127.73) (width 0.2) (layer F.Cu) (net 4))
 (segment (start 161.0987 128.7989) (end 156.9889 128.7989) (width 0.2) (layer F.Cu) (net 4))
 (segment (start 162.27 129.9702) (end 161.0987 128.7989) (width 0.2) (layer F.Cu) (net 4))
 (segment (start 162.27 130.5634) (end 162.27 129.9702) (width 0.2) (layer F.Cu) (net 4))
 (segment (start 163.915 132.2084) (end 162.27 130.5634) (width 0.2) (layer F.Cu) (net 4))
 (segment (start 165.907 132.2084) (end 163.915 132.2084) (width 0.2) (layer F.Cu) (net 4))
 (segment (start 172.5411 138.8425) (end 165.907 132.2084) (width 0.2) (layer F.Cu) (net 4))
 (segment (start 172.5411 144.2414) (end 172.5411 138.8425) (width 0.2) (layer F.Cu) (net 4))
 (segment (start 177.2446 148.9449) (end 172.5411 144.2414) (width 0.2) (layer F.Cu) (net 4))
 (segment (start 178.2353 148.9449) (end 177.2446 148.9449) (width 0.2) (layer F.Cu) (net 4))
 (segment (start 180.2904 151) (end 178.2353 148.9449) (width 0.2) (layer F.Cu) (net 4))
 (segment (start 190.35 151) (end 180.2904 151) (width 0.2) (layer F.Cu) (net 4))
 (segment (start 174.4086 177.1386) (end 173.27 176) (width 0.2) (layer F.Cu) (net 3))
 (segment (start 185.1314 177.1386) (end 174.4086 177.1386) (width 0.2) (layer F.Cu) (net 3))
 (segment (start 186.27 176) (end 185.1314 177.1386) (width 0.2) (layer F.Cu) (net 3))
 (segment (start 195.73 163.27) (end 195.73 164.2688) (width 0.2) (layer F.Cu) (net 3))
 (segment (start 173.54 143.81) (end 173.54 136.19) (width 0.2) (layer F.Cu) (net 3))
 (segment (start 152.9526 126.6536) (end 151.3581 128.2481) (width 0.2) (layer F.Cu) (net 3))
 (segment (start 161.4337 126.6536) (end 152.9526 126.6536) (width 0.2) (layer F.Cu) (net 3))
 (segment (start 162.27 127.4899) (end 161.4337 126.6536) (width 0.2) (layer F.Cu) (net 3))
 (segment (start 162.27 128.0069) (end 162.27 127.4899) (width 0.2) (layer F.Cu) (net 3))
 (segment (start 163.4707 129.2076) (end 162.27 128.0069) (width 0.2) (layer F.Cu) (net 3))
 (segment (start 164.0234 129.2076) (end 163.4707 129.2076) (width 0.2) (layer F.Cu) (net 3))
 (segment (start 164.81 129.9942) (end 164.0234 129.2076) (width 0.2) (layer F.Cu) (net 3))
 (segment (start 164.81 130.5105) (end 164.81 129.9942) (width 0.2) (layer F.Cu) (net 3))
 (segment (start 170.4895 136.19) (end 164.81 130.5105) (width 0.2) (layer F.Cu) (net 3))
 (segment (start 173.54 136.19) (end 170.4895 136.19) (width 0.2) (layer F.Cu) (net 3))
 (segment (start 150.84 127.73) (end 151.3581 128.2481) (width 0.2) (layer F.Cu) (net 3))
 (segment (start 152.11 136.61) (end 153 137.5) (width 0.2) (layer F.Cu) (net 3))
 (segment (start 152.11 129) (end 152.11 136.61) (width 0.2) (layer F.Cu) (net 3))
 (segment (start 151.3581 128.2481) (end 152.11 129) (width 0.2) (layer F.Cu) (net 3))
 (segment (start 202.27 171.1552) (end 202.27 176) (width 0.2) (layer F.Cu) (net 3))
 (segment (start 205.4764 171.1552) (end 202.27 171.1552) (width 0.2) (layer F.Cu) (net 3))
 (segment (start 217.1701 159.4615) (end 205.4764 171.1552) (width 0.2) (layer F.Cu) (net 3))
 (segment (start 217.1701 141.3299) (end 217.1701 159.4615) (width 0.2) (layer F.Cu) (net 3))
 (segment (start 224.5 134) (end 217.1701 141.3299) (width 0.2) (layer F.Cu) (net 3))
 (segment (start 195.73 164.6152) (end 195.73 164.2688) (width 0.2) (layer F.Cu) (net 3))
 (segment (start 202.27 171.1552) (end 195.73 164.6152) (width 0.2) (layer F.Cu) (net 3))
 (segment (start 153.6386 177.1386) (end 153 176.5) (width 0.2) (layer F.Cu) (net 3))
 (segment (start 172.1314 177.1386) (end 153.6386 177.1386) (width 0.2) (layer F.Cu) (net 3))
 (segment (start 173.27 176) (end 172.1314 177.1386) (width 0.2) (layer F.Cu) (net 3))
 (segment (start 162.9583 155.2967) (end 161.89 156.365) (width 0.2) (layer F.Cu) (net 3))
 (segment (start 162.9583 153.3866) (end 162.9583 155.2967) (width 0.2) (layer F.Cu) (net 3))
 (segment (start 155.3623 145.7906) (end 162.9583 153.3866) (width 0.2) (layer F.Cu) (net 3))
 (segment (start 154.2273 145.7906) (end 155.3623 145.7906) (width 0.2) (layer F.Cu) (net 3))
 (segment (start 151.5494 143.1127) (end 154.2273 145.7906) (width 0.2) (layer F.Cu) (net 3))
 (segment (start 151.5494 138.9506) (end 151.5494 143.1127) (width 0.2) (layer F.Cu) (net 3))
 (segment (start 153 137.5) (end 151.5494 138.9506) (width 0.2) (layer F.Cu) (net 3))
 (segment (start 151.9159 170.8668) (end 160.2119 162.5708) (width 0.2) (layer F.Cu) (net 3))
 (segment (start 151.9159 175.4159) (end 151.9159 170.8668) (width 0.2) (layer F.Cu) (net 3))
 (segment (start 153 176.5) (end 151.9159 175.4159) (width 0.2) (layer F.Cu) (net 3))
 (segment (start 158.2914 160.6503) (end 160.2119 162.5708) (width 0.2) (layer F.Cu) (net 3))
 (segment (start 158.2914 159.7361) (end 158.2914 160.6503) (width 0.2) (layer F.Cu) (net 3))
 (segment (start 159.1868 158.8407) (end 158.2914 159.7361) (width 0.2) (layer F.Cu) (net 3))
 (segment (start 159.6522 158.8407) (end 159.1868 158.8407) (width 0.2) (layer F.Cu) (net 3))
 (segment (start 161.89 156.6029) (end 159.6522 158.8407) (width 0.2) (layer F.Cu) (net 3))
 (segment (start 161.89 156.365) (end 161.89 156.6029) (width 0.2) (layer F.Cu) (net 3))
 (segment (start 170.0792 162.5708) (end 177.65 155) (width 0.2) (layer F.Cu) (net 3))
 (segment (start 160.2119 162.5708) (end 170.0792 162.5708) (width 0.2) (layer F.Cu) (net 3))
 (segment (start 186.27 176) (end 191.73 176) (width 0.2) (layer F.Cu) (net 3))
 (segment (start 200.7147 177.5553) (end 202.27 176) (width 0.2) (layer F.Cu) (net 3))
 (segment (start 193.2853 177.5553) (end 200.7147 177.5553) (width 0.2) (layer F.Cu) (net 3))
 (segment (start 191.73 176) (end 193.2853 177.5553) (width 0.2) (layer F.Cu) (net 3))
 (segment (start 213.9996 151.0004) (end 210 155) (width 0.2) (layer F.Cu) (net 13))
 (segment (start 213.9996 139.5004) (end 213.9996 151.0004) (width 0.2) (layer F.Cu) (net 13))
 (segment (start 219.5 134) (end 213.9996 139.5004) (width 0.2) (layer F.Cu) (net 13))
 (segment (start 205 170.08) (end 205 161.3914) (width 0.2) (layer F.Cu) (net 11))
 (segment (start 205.5317 161.3914) (end 205 161.3914) (width 0.2) (layer F.Cu) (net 11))
 (segment (start 207.572 159.3511) (end 205.5317 161.3914) (width 0.2) (layer F.Cu) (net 11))
 (segment (start 207.572 145.428) (end 207.572 159.3511) (width 0.2) (layer F.Cu) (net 11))
 (segment (start 210 143) (end 207.572 145.428) (width 0.2) (layer F.Cu) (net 11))
 (segment (start 198.9314 161.3914) (end 198.27 160.73) (width 0.2) (layer F.Cu) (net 11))
 (segment (start 205 161.3914) (end 198.9314 161.3914) (width 0.2) (layer F.Cu) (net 11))
 (segment (start 196.5801 140.7699) (end 198 139.35) (width 0.2) (layer F.Cu) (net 17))
 (segment (start 196.5801 160.4526) (end 196.5801 140.7699) (width 0.2) (layer F.Cu) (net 17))
 (segment (start 198.2692 162.1417) (end 196.5801 160.4526) (width 0.2) (layer F.Cu) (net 17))
 (segment (start 198.5543 162.1417) (end 198.2692 162.1417) (width 0.2) (layer F.Cu) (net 17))
 (segment (start 199.3406 162.928) (end 198.5543 162.1417) (width 0.2) (layer F.Cu) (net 17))
 (segment (start 199.3406 163.6136) (end 199.3406 162.928) (width 0.2) (layer F.Cu) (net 17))
 (segment (start 198.6552 164.299) (end 199.3406 163.6136) (width 0.2) (layer F.Cu) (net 17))
 (segment (start 197.8658 164.299) (end 198.6552 164.299) (width 0.2) (layer F.Cu) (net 17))
 (segment (start 196.7289 163.1621) (end 197.8658 164.299) (width 0.2) (layer F.Cu) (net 17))
 (segment (start 196.7289 162.3883) (end 196.7289 163.1621) (width 0.2) (layer F.Cu) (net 17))
 (segment (start 196.6018 162.2612) (end 196.7289 162.3883) (width 0.2) (layer F.Cu) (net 17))
 (segment (start 194.8336 162.2612) (end 196.6018 162.2612) (width 0.2) (layer F.Cu) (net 17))
 (segment (start 194.27 162.8248) (end 194.8336 162.2612) (width 0.2) (layer F.Cu) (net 17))
 (segment (start 194.27 176) (end 194.27 162.8248) (width 0.2) (layer F.Cu) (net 17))
 (segment (start 192.2681 167.4619) (end 183.73 176) (width 0.2) (layer F.Cu) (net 18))
 (segment (start 192.2681 150.2416) (end 192.2681 167.4619) (width 0.2) (layer F.Cu) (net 18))
 (segment (start 190.9354 148.9089) (end 192.2681 150.2416) (width 0.2) (layer F.Cu) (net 18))
 (segment (start 189.5589 148.9089) (end 190.9354 148.9089) (width 0.2) (layer F.Cu) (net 18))
 (segment (start 180 139.35) (end 189.5589 148.9089) (width 0.2) (layer F.Cu) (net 18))
 (segment (start 189.2708 144.0792) (end 190.35 143) (width 0.2) (layer F.Cu) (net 16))
 (segment (start 189.2708 147.4316) (end 189.2708 144.0792) (width 0.2) (layer F.Cu) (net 16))
 (segment (start 190.2663 148.4271) (end 189.2708 147.4316) (width 0.2) (layer F.Cu) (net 16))
 (segment (start 191.0476 148.4271) (end 190.2663 148.4271) (width 0.2) (layer F.Cu) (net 16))
 (segment (start 192.9811 150.3606) (end 191.0476 148.4271) (width 0.2) (layer F.Cu) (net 16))
 (segment (start 192.9811 176.3259) (end 192.9811 150.3606) (width 0.2) (layer F.Cu) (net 16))
 (segment (start 193.8101 177.1549) (end 192.9811 176.3259) (width 0.2) (layer F.Cu) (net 16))
 (segment (start 198.5751 177.1549) (end 193.8101 177.1549) (width 0.2) (layer F.Cu) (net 16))
 (segment (start 199.73 176) (end 198.5751 177.1549) (width 0.2) (layer F.Cu) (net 16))
 (segment (start 170.73 169.92) (end 177.65 163) (width 0.2) (layer F.Cu) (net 15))
 (segment (start 170.73 176) (end 170.73 169.92) (width 0.2) (layer F.Cu) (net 15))
 (segment (start 193.3815 158.3815) (end 198.27 163.27) (width 0.2) (layer F.Cu) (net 10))
 (segment (start 193.3815 150.0315) (end 193.3815 158.3815) (width 0.2) (layer F.Cu) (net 10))
 (segment (start 190.35 147) (end 193.3815 150.0315) (width 0.2) (layer F.Cu) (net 10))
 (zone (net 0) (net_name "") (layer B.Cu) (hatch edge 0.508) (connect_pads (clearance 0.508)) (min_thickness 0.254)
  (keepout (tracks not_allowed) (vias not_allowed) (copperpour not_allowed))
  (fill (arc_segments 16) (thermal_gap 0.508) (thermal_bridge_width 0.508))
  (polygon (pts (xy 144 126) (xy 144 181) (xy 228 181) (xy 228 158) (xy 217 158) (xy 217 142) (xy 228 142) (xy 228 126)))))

